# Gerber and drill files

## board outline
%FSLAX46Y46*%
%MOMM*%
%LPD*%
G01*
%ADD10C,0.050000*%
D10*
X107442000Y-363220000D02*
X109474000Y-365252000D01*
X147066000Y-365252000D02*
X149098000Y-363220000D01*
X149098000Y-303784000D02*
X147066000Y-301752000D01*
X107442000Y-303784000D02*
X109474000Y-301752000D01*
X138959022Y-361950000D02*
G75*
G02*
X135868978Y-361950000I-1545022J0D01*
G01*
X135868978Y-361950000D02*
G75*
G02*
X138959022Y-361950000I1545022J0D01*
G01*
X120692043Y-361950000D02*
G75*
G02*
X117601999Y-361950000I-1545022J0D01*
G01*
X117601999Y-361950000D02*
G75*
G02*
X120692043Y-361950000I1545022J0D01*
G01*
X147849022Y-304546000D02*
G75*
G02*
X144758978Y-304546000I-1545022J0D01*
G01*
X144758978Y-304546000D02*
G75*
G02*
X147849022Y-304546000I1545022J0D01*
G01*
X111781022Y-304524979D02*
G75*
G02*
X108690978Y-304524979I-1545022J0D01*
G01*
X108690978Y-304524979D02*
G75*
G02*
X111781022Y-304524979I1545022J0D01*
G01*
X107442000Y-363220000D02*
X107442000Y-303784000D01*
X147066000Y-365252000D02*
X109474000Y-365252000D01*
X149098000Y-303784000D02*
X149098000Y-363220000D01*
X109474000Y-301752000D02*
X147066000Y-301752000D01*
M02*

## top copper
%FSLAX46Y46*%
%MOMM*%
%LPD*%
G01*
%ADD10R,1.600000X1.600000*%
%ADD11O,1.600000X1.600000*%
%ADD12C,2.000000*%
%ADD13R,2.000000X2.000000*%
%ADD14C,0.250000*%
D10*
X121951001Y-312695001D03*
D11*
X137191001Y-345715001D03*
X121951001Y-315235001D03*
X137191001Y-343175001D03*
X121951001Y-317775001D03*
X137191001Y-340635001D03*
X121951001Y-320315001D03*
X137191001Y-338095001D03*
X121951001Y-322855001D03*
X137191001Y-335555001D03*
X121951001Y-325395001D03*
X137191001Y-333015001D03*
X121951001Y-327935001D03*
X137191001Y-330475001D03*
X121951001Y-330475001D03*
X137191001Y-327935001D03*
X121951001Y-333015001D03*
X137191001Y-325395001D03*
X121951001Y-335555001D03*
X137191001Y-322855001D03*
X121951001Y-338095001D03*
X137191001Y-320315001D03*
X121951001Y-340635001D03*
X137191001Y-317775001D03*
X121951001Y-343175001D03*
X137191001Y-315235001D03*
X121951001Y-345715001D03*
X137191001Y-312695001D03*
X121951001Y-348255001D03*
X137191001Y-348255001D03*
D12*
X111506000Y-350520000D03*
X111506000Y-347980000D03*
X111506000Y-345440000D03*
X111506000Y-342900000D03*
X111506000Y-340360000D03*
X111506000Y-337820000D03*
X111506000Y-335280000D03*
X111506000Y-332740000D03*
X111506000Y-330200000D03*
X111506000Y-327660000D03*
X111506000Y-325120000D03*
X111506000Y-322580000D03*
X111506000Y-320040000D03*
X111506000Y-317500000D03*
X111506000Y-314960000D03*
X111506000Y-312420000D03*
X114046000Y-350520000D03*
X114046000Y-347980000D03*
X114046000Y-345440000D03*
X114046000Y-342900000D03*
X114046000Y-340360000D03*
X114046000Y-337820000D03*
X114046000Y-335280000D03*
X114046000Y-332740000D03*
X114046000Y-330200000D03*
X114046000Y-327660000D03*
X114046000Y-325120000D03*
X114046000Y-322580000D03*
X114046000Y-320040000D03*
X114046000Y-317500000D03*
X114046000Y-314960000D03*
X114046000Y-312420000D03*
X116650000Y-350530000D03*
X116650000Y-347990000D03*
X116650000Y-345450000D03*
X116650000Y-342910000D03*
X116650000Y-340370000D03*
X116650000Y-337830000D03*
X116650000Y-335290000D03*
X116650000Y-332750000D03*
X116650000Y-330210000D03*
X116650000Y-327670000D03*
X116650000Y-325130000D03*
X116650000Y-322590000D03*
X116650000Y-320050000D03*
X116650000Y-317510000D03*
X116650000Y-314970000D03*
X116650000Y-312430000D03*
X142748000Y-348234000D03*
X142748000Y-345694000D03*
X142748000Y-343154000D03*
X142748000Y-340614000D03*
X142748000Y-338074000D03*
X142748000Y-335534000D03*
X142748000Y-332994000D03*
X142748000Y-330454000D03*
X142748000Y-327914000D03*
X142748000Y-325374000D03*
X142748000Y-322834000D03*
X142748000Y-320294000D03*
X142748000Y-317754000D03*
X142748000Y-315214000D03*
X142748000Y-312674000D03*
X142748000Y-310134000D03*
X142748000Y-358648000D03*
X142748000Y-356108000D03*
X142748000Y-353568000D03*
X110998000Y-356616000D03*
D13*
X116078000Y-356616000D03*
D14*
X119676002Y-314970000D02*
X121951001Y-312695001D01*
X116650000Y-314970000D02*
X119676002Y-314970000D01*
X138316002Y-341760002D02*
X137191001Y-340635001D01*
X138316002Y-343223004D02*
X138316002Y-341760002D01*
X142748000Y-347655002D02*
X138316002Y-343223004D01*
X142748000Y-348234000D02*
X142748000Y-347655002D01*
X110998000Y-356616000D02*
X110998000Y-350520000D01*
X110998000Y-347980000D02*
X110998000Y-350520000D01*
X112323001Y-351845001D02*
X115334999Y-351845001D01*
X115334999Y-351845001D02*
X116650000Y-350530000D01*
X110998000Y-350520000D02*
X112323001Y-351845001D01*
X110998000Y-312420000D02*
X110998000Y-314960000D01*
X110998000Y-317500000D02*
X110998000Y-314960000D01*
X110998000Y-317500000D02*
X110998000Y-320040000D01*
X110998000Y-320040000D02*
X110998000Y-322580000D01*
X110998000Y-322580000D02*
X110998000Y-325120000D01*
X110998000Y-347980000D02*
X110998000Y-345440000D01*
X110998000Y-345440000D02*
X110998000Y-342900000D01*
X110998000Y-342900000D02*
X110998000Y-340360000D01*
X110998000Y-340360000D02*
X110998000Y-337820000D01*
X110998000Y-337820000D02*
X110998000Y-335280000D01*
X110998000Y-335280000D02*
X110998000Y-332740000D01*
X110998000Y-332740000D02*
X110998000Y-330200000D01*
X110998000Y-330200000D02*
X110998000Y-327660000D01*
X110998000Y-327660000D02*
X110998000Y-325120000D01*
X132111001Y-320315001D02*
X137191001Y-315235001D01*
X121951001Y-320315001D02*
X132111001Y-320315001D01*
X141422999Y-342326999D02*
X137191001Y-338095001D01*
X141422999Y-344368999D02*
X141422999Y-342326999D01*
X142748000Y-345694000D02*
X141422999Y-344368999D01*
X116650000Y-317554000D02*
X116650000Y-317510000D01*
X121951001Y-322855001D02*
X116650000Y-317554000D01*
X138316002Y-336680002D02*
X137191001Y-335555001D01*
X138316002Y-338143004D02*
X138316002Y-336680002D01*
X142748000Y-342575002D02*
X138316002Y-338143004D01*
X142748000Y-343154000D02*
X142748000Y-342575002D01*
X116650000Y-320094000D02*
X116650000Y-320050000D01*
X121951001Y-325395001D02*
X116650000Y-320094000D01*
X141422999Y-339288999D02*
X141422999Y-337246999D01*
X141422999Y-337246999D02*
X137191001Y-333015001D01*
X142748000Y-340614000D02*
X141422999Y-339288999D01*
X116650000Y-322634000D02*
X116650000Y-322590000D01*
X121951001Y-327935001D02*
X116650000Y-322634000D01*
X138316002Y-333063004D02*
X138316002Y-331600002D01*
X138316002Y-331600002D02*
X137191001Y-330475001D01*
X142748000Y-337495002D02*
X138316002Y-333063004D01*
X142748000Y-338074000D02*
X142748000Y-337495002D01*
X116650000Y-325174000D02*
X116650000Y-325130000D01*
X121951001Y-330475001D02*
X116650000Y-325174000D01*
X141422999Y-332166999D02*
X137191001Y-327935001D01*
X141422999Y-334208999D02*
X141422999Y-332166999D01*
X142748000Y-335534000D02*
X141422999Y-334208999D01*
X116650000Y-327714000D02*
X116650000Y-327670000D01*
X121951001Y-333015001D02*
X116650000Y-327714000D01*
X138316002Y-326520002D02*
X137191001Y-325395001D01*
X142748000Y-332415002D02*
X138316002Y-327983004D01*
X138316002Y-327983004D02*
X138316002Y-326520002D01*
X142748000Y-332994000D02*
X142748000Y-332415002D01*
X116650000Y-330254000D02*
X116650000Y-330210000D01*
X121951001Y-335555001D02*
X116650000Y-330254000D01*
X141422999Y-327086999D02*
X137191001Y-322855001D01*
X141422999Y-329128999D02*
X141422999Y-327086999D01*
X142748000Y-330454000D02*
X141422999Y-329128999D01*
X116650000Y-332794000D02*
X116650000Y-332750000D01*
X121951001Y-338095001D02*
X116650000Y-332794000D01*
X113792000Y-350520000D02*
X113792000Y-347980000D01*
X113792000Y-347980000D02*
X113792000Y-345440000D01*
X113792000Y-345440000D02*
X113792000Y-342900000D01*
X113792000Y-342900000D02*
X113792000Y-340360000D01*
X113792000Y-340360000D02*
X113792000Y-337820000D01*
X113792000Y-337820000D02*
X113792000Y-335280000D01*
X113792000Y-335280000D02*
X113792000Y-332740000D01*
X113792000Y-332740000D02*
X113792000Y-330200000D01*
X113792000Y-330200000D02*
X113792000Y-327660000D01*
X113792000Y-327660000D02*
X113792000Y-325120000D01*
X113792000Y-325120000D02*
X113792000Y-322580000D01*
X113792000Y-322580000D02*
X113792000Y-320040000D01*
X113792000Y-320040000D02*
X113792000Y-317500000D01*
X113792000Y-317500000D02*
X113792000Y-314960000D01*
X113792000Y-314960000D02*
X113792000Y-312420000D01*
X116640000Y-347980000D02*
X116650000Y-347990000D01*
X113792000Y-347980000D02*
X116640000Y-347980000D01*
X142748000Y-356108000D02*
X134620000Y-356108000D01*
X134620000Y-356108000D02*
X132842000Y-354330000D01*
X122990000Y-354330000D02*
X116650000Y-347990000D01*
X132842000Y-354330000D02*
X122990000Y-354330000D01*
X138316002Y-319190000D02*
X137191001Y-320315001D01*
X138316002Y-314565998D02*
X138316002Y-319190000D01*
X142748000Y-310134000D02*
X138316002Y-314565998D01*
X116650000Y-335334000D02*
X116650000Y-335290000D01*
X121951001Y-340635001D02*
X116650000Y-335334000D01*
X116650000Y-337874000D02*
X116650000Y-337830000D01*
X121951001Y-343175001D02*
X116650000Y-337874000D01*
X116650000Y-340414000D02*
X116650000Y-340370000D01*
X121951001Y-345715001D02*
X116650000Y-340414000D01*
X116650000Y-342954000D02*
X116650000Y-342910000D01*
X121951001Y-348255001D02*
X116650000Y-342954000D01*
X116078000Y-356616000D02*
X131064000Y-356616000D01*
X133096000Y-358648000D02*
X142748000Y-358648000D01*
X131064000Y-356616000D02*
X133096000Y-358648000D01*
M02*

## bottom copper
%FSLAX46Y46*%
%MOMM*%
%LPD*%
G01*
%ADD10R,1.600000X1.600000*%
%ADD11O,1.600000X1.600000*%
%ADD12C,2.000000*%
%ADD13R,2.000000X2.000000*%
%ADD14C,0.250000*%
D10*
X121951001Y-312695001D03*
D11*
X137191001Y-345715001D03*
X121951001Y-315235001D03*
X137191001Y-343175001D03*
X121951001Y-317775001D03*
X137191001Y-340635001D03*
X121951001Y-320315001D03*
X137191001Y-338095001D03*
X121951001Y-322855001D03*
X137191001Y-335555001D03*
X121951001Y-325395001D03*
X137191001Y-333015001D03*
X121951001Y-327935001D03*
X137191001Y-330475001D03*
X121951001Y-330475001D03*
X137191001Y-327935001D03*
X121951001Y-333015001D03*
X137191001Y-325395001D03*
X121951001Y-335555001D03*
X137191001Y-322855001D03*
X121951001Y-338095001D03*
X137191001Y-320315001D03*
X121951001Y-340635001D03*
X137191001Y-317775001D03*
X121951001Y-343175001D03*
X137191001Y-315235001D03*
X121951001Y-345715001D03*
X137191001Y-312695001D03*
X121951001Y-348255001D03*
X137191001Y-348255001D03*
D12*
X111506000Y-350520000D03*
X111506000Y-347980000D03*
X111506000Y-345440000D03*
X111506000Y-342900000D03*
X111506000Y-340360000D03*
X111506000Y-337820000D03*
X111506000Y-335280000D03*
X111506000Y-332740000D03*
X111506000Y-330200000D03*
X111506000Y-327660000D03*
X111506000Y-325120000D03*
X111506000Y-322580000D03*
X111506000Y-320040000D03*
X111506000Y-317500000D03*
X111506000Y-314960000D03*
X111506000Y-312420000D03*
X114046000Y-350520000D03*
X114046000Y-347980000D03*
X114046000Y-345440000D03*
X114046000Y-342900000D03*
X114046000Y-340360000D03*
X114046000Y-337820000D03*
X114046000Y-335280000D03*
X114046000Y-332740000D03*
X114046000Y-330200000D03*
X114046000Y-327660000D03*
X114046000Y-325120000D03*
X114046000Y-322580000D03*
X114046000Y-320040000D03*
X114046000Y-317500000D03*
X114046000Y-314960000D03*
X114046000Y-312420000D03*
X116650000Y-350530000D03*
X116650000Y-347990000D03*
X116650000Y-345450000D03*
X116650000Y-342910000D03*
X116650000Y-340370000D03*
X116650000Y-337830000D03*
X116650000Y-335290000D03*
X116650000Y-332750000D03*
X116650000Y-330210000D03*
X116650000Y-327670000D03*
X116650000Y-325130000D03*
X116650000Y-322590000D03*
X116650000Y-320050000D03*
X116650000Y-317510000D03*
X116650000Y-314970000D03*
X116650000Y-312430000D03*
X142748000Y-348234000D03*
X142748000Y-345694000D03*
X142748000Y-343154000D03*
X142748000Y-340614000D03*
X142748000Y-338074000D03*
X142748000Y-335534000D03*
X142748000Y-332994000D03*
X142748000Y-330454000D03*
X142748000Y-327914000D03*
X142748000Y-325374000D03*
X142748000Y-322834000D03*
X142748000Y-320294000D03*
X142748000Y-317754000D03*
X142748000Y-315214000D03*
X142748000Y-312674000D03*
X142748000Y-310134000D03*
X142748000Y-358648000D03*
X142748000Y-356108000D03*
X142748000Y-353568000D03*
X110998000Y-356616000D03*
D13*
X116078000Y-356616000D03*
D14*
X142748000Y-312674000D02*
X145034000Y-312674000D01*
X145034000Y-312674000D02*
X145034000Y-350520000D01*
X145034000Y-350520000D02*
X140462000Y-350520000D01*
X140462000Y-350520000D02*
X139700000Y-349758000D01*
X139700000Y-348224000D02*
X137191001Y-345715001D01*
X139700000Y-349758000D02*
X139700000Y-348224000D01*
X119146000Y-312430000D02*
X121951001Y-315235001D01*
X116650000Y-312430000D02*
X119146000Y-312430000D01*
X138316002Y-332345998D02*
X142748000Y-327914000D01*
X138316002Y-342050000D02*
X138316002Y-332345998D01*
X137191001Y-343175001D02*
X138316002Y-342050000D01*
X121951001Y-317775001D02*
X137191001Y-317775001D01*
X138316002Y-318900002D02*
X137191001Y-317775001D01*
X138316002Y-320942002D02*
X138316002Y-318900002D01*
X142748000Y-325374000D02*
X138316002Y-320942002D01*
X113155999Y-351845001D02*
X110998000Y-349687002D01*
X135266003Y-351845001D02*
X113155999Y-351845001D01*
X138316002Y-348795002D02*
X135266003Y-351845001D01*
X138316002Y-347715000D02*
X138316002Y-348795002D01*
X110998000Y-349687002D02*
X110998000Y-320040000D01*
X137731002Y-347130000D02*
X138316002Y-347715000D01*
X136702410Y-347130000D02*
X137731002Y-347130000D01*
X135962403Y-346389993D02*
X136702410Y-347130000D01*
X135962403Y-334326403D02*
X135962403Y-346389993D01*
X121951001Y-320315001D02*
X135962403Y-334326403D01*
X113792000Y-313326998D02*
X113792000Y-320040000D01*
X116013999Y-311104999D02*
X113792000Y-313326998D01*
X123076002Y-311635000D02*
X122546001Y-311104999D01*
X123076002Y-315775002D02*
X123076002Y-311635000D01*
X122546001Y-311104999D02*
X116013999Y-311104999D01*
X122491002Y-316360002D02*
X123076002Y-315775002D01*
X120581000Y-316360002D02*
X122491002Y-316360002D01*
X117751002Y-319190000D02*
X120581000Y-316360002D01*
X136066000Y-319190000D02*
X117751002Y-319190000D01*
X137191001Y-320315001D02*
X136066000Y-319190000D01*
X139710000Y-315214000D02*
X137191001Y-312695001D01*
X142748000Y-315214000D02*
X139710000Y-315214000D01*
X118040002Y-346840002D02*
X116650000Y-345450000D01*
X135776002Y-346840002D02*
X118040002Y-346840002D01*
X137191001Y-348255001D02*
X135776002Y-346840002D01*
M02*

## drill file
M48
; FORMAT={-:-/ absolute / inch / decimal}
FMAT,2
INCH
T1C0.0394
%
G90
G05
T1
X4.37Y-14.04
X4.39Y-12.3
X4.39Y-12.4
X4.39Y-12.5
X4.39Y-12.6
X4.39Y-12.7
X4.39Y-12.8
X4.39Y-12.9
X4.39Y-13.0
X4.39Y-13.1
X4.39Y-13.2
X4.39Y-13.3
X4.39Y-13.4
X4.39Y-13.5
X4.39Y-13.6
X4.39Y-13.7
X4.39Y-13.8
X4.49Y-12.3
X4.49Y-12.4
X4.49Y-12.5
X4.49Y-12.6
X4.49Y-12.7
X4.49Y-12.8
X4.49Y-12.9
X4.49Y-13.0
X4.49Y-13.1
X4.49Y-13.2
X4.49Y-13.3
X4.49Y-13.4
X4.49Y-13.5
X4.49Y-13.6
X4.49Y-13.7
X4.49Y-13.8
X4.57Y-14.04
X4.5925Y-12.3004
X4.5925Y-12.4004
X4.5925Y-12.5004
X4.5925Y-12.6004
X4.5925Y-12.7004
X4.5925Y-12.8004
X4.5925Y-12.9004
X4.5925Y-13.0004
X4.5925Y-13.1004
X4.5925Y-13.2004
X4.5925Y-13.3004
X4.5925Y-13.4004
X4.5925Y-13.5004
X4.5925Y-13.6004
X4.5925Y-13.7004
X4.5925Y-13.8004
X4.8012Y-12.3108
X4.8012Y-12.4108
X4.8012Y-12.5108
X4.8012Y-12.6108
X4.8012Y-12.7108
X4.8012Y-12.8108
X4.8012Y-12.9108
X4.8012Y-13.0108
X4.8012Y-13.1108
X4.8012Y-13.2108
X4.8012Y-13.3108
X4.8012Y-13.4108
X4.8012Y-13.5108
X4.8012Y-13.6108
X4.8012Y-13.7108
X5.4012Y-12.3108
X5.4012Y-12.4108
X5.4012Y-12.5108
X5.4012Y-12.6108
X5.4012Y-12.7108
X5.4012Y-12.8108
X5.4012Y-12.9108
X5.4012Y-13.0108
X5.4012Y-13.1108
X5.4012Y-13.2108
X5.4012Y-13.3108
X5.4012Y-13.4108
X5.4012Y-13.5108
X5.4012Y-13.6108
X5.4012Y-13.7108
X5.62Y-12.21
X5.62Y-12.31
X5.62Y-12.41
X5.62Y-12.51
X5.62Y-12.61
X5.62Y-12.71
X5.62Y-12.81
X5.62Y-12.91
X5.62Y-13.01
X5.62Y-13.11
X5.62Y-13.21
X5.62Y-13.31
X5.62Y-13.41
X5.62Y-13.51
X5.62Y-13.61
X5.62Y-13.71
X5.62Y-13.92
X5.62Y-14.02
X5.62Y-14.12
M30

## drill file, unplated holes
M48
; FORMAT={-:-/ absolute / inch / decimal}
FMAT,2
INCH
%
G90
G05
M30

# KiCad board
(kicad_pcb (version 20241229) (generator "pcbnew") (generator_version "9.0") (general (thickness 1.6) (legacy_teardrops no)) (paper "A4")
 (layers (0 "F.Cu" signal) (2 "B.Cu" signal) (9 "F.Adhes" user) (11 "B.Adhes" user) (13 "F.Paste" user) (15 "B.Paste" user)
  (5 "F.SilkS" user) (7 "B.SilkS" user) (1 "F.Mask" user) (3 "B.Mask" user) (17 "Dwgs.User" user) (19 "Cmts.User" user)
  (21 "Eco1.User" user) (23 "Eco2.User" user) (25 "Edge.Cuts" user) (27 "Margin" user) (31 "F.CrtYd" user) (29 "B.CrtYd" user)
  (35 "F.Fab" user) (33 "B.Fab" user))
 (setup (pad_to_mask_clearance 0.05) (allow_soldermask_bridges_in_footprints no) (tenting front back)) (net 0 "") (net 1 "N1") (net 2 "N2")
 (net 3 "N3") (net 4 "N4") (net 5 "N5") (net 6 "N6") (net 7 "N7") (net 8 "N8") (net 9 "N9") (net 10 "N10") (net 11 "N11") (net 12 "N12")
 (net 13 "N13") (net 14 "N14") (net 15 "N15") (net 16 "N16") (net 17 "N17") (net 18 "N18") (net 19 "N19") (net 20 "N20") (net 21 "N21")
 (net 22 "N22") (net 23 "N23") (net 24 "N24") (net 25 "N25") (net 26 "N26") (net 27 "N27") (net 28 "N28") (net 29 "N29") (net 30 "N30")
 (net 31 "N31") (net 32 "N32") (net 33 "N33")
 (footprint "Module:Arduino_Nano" (layer "F.Cu") (at 121.951001 312.695001)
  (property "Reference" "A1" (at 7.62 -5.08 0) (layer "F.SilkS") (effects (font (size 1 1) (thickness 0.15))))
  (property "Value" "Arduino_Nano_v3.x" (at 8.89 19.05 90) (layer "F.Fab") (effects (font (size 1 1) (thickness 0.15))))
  (pad "1" thru_hole rect (at 0 0) (size 1.6 1.6) (drill 1) (layers "*.Cu" "*.Mask") (remove_unused_layers no) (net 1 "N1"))
  (pad "2" thru_hole oval (at 0 2.54) (size 1.6 1.6) (drill 1) (layers "*.Cu" "*.Mask") (remove_unused_layers no) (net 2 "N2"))
  (pad "3" thru_hole oval (at 0 5.08) (size 1.6 1.6) (drill 1) (layers "*.Cu" "*.Mask") (remove_unused_layers no) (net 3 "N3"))
  (pad "4" thru_hole oval (at 0 7.62) (size 1.6 1.6) (drill 1) (layers "*.Cu" "*.Mask") (remove_unused_layers no) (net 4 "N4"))
  (pad "5" thru_hole oval (at 0 10.16) (size 1.6 1.6) (drill 1) (layers "*.Cu" "*.Mask") (remove_unused_layers no) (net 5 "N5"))
  (pad "6" thru_hole oval (at 0 12.7) (size 1.6 1.6) (drill 1) (layers "*.Cu" "*.Mask") (remove_unused_layers no) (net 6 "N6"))
  (pad "7" thru_hole oval (at 0 15.24) (size 1.6 1.6) (drill 1) (layers "*.Cu" "*.Mask") (remove_unused_layers no) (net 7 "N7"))
  (pad "8" thru_hole oval (at 0 17.78) (size 1.6 1.6) (drill 1) (layers "*.Cu" "*.Mask") (remove_unused_layers no) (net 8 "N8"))
  (pad "9" thru_hole oval (at 0 20.32) (size 1.6 1.6) (drill 1) (layers "*.Cu" "*.Mask") (remove_unused_layers no) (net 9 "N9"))
  (pad "10" thru_hole oval (at 0 22.86) (size 1.6 1.6) (drill 1) (layers "*.Cu" "*.Mask") (remove_unused_layers no) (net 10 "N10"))
  (pad "11" thru_hole oval (at 0 25.4) (size 1.6 1.6) (drill 1) (layers "*.Cu" "*.Mask") (remove_unused_layers no) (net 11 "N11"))
  (pad "12" thru_hole oval (at 0 27.94) (size 1.6 1.6) (drill 1) (layers "*.Cu" "*.Mask") (remove_unused_layers no) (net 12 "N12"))
  (pad "13" thru_hole oval (at 0 30.48) (size 1.6 1.6) (drill 1) (layers "*.Cu" "*.Mask") (remove_unused_layers no) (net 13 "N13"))
  (pad "14" thru_hole oval (at 0 33.02) (size 1.6 1.6) (drill 1) (layers "*.Cu" "*.Mask") (remove_unused_layers no) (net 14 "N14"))
  (pad "15" thru_hole oval (at 0 35.56) (size 1.6 1.6) (drill 1) (layers "*.Cu" "*.Mask") (remove_unused_layers no) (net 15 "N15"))
  (pad "16" thru_hole oval (at 15.24 35.56) (size 1.6 1.6) (drill 1) (layers "*.Cu" "*.Mask") (remove_unused_layers no) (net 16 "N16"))
  (pad "17" thru_hole oval (at 15.24 33.02) (size 1.6 1.6) (drill 1) (layers "*.Cu" "*.Mask") (remove_unused_layers no) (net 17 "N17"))
  (pad "18" thru_hole oval (at 15.24 30.48) (size 1.6 1.6) (drill 1) (layers "*.Cu" "*.Mask") (remove_unused_layers no) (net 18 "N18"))
  (pad "19" thru_hole oval (at 15.24 27.94) (size 1.6 1.6) (drill 1) (layers "*.Cu" "*.Mask") (remove_unused_layers no) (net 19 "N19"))
  (pad "20" thru_hole oval (at 15.24 25.4) (size 1.6 1.6) (drill 1) (layers "*.Cu" "*.Mask") (remove_unused_layers no) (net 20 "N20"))
  (pad "21" thru_hole oval (at 15.24 22.86) (size 1.6 1.6) (drill 1) (layers "*.Cu" "*.Mask") (remove_unused_layers no) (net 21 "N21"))
  (pad "22" thru_hole oval (at 15.24 20.32) (size 1.6 1.6) (drill 1) (layers "*.Cu" "*.Mask") (remove_unused_layers no) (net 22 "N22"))
  (pad "23" thru_hole oval (at 15.24 17.78) (size 1.6 1.6) (drill 1) (layers "*.Cu" "*.Mask") (remove_unused_layers no) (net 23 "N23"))
  (pad "24" thru_hole oval (at 15.24 15.24) (size 1.6 1.6) (drill 1) (layers "*.Cu" "*.Mask") (remove_unused_layers no) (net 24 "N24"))
  (pad "25" thru_hole oval (at 15.24 12.7) (size 1.6 1.6) (drill 1) (layers "*.Cu" "*.Mask") (remove_unused_layers no) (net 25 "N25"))
  (pad "26" thru_hole oval (at 15.24 10.16) (size 1.6 1.6) (drill 1) (layers "*.Cu" "*.Mask") (remove_unused_layers no) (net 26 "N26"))
  (pad "27" thru_hole oval (at 15.24 7.62) (size 1.6 1.6) (drill 1) (layers "*.Cu" "*.Mask") (remove_unused_layers no) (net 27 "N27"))
  (pad "28" thru_hole oval (at 15.24 5.08) (size 1.6 1.6) (drill 1) (layers "*.Cu" "*.Mask") (remove_unused_layers no) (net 3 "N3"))
  (pad "29" thru_hole oval (at 15.24 2.54) (size 1.6 1.6) (drill 1) (layers "*.Cu" "*.Mask") (remove_unused_layers no) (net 4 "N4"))
  (pad "30" thru_hole oval (at 15.24 0) (size 1.6 1.6) (drill 1) (layers "*.Cu" "*.Mask") (remove_unused_layers no) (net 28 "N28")))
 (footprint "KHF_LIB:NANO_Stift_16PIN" (layer "F.Cu") (at 114.046 312.42 -90)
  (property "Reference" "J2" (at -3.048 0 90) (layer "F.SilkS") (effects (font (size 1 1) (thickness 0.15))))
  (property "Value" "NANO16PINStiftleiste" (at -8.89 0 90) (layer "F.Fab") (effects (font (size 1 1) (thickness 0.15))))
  (pad "1" thru_hole circle (at 0 0 270) (size 2 2) (drill 1) (layers "*.Cu" "*.Mask") (remove_unused_layers no) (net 27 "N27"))
  (pad "2" thru_hole circle (at 2.54 0 270) (size 2 2) (drill 1) (layers "*.Cu" "*.Mask") (remove_unused_layers no) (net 27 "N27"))
  (pad "3" thru_hole circle (at 5.08 0 270) (size 2 2) (drill 1) (layers "*.Cu" "*.Mask") (remove_unused_layers no) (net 27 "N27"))
  (pad "4" thru_hole circle (at 7.62 0 270) (size 2 2) (drill 1) (layers "*.Cu" "*.Mask") (remove_unused_layers no) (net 27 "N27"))
  (pad "5" thru_hole circle (at 10.16 0 270) (size 2 2) (drill 1) (layers "*.Cu" "*.Mask") (remove_unused_layers no) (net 27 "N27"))
  (pad "6" thru_hole circle (at 12.7 0 270) (size 2 2) (drill 1) (layers "*.Cu" "*.Mask") (remove_unused_layers no) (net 27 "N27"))
  (pad "7" thru_hole circle (at 15.24 0 270) (size 2 2) (drill 1) (layers "*.Cu" "*.Mask") (remove_unused_layers no) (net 27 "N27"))
  (pad "8" thru_hole circle (at 17.78 0 270) (size 2 2) (drill 1) (layers "*.Cu" "*.Mask") (remove_unused_layers no) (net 27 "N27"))
  (pad "9" thru_hole circle (at 20.32 0 270) (size 2 2) (drill 1) (layers "*.Cu" "*.Mask") (remove_unused_layers no) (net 27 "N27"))
  (pad "10" thru_hole circle (at 22.86 0 270) (size 2 2) (drill 1) (layers "*.Cu" "*.Mask") (remove_unused_layers no) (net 27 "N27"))
  (pad "11" thru_hole circle (at 25.4 0 270) (size 2 2) (drill 1) (layers "*.Cu" "*.Mask") (remove_unused_layers no) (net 27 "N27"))
  (pad "12" thru_hole circle (at 27.94 0 270) (size 2 2) (drill 1) (layers "*.Cu" "*.Mask") (remove_unused_layers no) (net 27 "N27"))
  (pad "13" thru_hole circle (at 30.48 0 270) (size 2 2) (drill 1) (layers "*.Cu" "*.Mask") (remove_unused_layers no) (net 27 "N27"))
  (pad "14" thru_hole circle (at 33.02 0 270) (size 2 2) (drill 1) (layers "*.Cu" "*.Mask") (remove_unused_layers no) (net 27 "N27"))
  (pad "15" thru_hole circle (at 35.56 0 270) (size 2 2) (drill 1) (layers "*.Cu" "*.Mask") (remove_unused_layers no) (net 27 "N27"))
  (pad "16" thru_hole circle (at 38.1 0 270) (size 2 2) (drill 1) (layers "*.Cu" "*.Mask") (remove_unused_layers no) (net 27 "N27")))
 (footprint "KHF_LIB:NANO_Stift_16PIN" (layer "F.Cu") (at 116.65 312.43 -90)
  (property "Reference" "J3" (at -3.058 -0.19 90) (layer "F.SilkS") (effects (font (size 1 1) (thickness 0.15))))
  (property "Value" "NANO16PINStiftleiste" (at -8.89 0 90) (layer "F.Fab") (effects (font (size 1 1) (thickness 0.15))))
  (pad "1" thru_hole circle (at 0 0 270) (size 2 2) (drill 1) (layers "*.Cu" "*.Mask") (remove_unused_layers no) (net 2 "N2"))
  (pad "2" thru_hole circle (at 2.54 0 270) (size 2 2) (drill 1) (layers "*.Cu" "*.Mask") (remove_unused_layers no) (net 1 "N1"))
  (pad "3" thru_hole circle (at 5.08 0 270) (size 2 2) (drill 1) (layers "*.Cu" "*.Mask") (remove_unused_layers no) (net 5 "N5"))
  (pad "4" thru_hole circle (at 7.62 0 270) (size 2 2) (drill 1) (layers "*.Cu" "*.Mask") (remove_unused_layers no) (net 6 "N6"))
  (pad "5" thru_hole circle (at 10.16 0 270) (size 2 2) (drill 1) (layers "*.Cu" "*.Mask") (remove_unused_layers no) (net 7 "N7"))
  (pad "6" thru_hole circle (at 12.7 0 270) (size 2 2) (drill 1) (layers "*.Cu" "*.Mask") (remove_unused_layers no) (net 8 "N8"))
  (pad "7" thru_hole circle (at 15.24 0 270) (size 2 2) (drill 1) (layers "*.Cu" "*.Mask") (remove_unused_layers no) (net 9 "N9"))
  (pad "8" thru_hole circle (at 17.78 0 270) (size 2 2) (drill 1) (layers "*.Cu" "*.Mask") (remove_unused_layers no) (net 10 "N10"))
  (pad "9" thru_hole circle (at 20.32 0 270) (size 2 2) (drill 1) (layers "*.Cu" "*.Mask") (remove_unused_layers no) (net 11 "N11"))
  (pad "10" thru_hole circle (at 22.86 0 270) (size 2 2) (drill 1) (layers "*.Cu" "*.Mask") (remove_unused_layers no) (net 12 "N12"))
  (pad "11" thru_hole circle (at 25.4 0 270) (size 2 2) (drill 1) (layers "*.Cu" "*.Mask") (remove_unused_layers no) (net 13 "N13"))
  (pad "12" thru_hole circle (at 27.94 0 270) (size 2 2) (drill 1) (layers "*.Cu" "*.Mask") (remove_unused_layers no) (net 14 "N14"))
  (pad "13" thru_hole circle (at 30.48 0 270) (size 2 2) (drill 1) (layers "*.Cu" "*.Mask") (remove_unused_layers no) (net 15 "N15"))
  (pad "14" thru_hole circle (at 33.02 0 270) (size 2 2) (drill 1) (layers "*.Cu" "*.Mask") (remove_unused_layers no) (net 16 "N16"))
  (pad "15" thru_hole circle (at 35.56 0 270) (size 2 2) (drill 1) (layers "*.Cu" "*.Mask") (remove_unused_layers no) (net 27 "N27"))
  (pad "16" thru_hole circle (at 38.1 0 270) (size 2 2) (drill 1) (layers "*.Cu" "*.Mask") (remove_unused_layers no) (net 4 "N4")))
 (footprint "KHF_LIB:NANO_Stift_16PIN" (layer "F.Cu") (at 142.748 348.234 90)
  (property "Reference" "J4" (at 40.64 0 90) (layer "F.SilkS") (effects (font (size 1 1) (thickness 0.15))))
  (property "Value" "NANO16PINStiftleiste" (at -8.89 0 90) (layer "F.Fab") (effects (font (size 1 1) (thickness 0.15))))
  (pad "1" thru_hole circle (at 0 0 90) (size 2 2) (drill 1) (layers "*.Cu" "*.Mask") (remove_unused_layers no) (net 19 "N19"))
  (pad "2" thru_hole circle (at 2.54 0 90) (size 2 2) (drill 1) (layers "*.Cu" "*.Mask") (remove_unused_layers no) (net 20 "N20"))
  (pad "3" thru_hole circle (at 5.08 0 90) (size 2 2) (drill 1) (layers "*.Cu" "*.Mask") (remove_unused_layers no) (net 21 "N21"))
  (pad "4" thru_hole circle (at 7.62 0 90) (size 2 2) (drill 1) (layers "*.Cu" "*.Mask") (remove_unused_layers no) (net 22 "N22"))
  (pad "5" thru_hole circle (at 10.16 0 90) (size 2 2) (drill 1) (layers "*.Cu" "*.Mask") (remove_unused_layers no) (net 23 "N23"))
  (pad "6" thru_hole circle (at 12.7 0 90) (size 2 2) (drill 1) (layers "*.Cu" "*.Mask") (remove_unused_layers no) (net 24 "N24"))
  (pad "7" thru_hole circle (at 15.24 0 90) (size 2 2) (drill 1) (layers "*.Cu" "*.Mask") (remove_unused_layers no) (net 25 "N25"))
  (pad "8" thru_hole circle (at 17.78 0 90) (size 2 2) (drill 1) (layers "*.Cu" "*.Mask") (remove_unused_layers no) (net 26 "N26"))
  (pad "9" thru_hole circle (at 20.32 0 90) (size 2 2) (drill 1) (layers "*.Cu" "*.Mask") (remove_unused_layers no) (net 18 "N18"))
  (pad "10" thru_hole circle (at 22.86 0 90) (size 2 2) (drill 1) (layers "*.Cu" "*.Mask") (remove_unused_layers no) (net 3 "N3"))
  (pad "11" thru_hole circle (at 25.4 0 90) (size 2 2) (drill 1) (layers "*.Cu" "*.Mask") (remove_unused_layers no) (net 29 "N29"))
  (pad "12" thru_hole circle (at 27.94 0 90) (size 2 2) (drill 1) (layers "*.Cu" "*.Mask") (remove_unused_layers no) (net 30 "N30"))
  (pad "13" thru_hole circle (at 30.48 0 90) (size 2 2) (drill 1) (layers "*.Cu" "*.Mask") (remove_unused_layers no) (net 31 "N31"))
  (pad "14" thru_hole circle (at 33.02 0 90) (size 2 2) (drill 1) (layers "*.Cu" "*.Mask") (remove_unused_layers no) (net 28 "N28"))
  (pad "15" thru_hole circle (at 35.56 0 90) (size 2 2) (drill 1) (layers "*.Cu" "*.Mask") (remove_unused_layers no) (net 17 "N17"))
  (pad "16" thru_hole circle (at 38.1 0 90) (size 2 2) (drill 1) (layers "*.Cu" "*.Mask") (remove_unused_layers no) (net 27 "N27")))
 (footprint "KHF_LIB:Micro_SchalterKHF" (layer "F.Cu") (at 142.748 358.648 90)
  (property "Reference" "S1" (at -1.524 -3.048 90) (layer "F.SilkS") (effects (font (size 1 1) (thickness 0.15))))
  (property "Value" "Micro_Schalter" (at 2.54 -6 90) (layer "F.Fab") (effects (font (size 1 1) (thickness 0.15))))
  (pad "1" thru_hole circle (at 0 0 90) (size 2 2) (drill 1) (layers "*.Cu" "*.Mask") (remove_unused_layers no) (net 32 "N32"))
  (pad "2" thru_hole circle (at 2.54 0 90) (size 2 2) (drill 1) (layers "*.Cu" "*.Mask") (remove_unused_layers no) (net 27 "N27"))
  (pad "3" thru_hole circle (at 5.08 0 90) (size 2 2) (drill 1) (layers "*.Cu" "*.Mask") (remove_unused_layers no) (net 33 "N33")))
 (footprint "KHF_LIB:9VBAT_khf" (layer "F.Cu") (at 110.998 356.616)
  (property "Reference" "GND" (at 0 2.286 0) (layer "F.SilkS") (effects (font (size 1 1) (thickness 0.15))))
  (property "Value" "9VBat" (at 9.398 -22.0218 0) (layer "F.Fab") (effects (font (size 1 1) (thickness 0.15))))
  (pad "1" thru_hole circle (at 0 0) (size 2 2) (drill 1) (layers "*.Cu" "*.Mask") (remove_unused_layers no) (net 4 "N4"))
  (pad "2" thru_hole rect (at 5.08 0) (size 2 2) (drill 1) (layers "*.Cu" "*.Mask") (remove_unused_layers no) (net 32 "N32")))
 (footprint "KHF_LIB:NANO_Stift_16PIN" (layer "F.Cu") (at 111.506 350.52 90)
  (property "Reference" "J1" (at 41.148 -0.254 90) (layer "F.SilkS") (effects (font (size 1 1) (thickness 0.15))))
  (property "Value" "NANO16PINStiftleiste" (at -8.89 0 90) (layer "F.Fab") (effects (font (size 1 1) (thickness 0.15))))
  (pad "1" thru_hole circle (at 0 0 90) (size 2 2) (drill 1) (layers "*.Cu" "*.Mask") (remove_unused_layers no) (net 4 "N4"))
  (pad "2" thru_hole circle (at 2.54 0 90) (size 2 2) (drill 1) (layers "*.Cu" "*.Mask") (remove_unused_layers no) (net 4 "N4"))
  (pad "3" thru_hole circle (at 5.08 0 90) (size 2 2) (drill 1) (layers "*.Cu" "*.Mask") (remove_unused_layers no) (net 4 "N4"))
  (pad "4" thru_hole circle (at 7.62 0 90) (size 2 2) (drill 1) (layers "*.Cu" "*.Mask") (remove_unused_layers no) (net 4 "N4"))
  (pad "5" thru_hole circle (at 10.16 0 90) (size 2 2) (drill 1) (layers "*.Cu" "*.Mask") (remove_unused_layers no) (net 4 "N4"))
  (pad "6" thru_hole circle (at 12.7 0 90) (size 2 2) (drill 1) (layers "*.Cu" "*.Mask") (remove_unused_layers no) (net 4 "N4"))
  (pad "7" thru_hole circle (at 15.24 0 90) (size 2 2) (drill 1) (layers "*.Cu" "*.Mask") (remove_unused_layers no) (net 4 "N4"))
  (pad "8" thru_hole circle (at 17.78 0 90) (size 2 2) (drill 1) (layers "*.Cu" "*.Mask") (remove_unused_layers no) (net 4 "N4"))
  (pad "9" thru_hole circle (at 20.32 0 90) (size 2 2) (drill 1) (layers "*.Cu" "*.Mask") (remove_unused_layers no) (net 4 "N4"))
  (pad "10" thru_hole circle (at 22.86 0 90) (size 2 2) (drill 1) (layers "*.Cu" "*.Mask") (remove_unused_layers no) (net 4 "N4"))
  (pad "11" thru_hole circle (at 25.4 0 90) (size 2 2) (drill 1) (layers "*.Cu" "*.Mask") (remove_unused_layers no) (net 4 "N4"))
  (pad "12" thru_hole circle (at 27.94 0 90) (size 2 2) (drill 1) (layers "*.Cu" "*.Mask") (remove_unused_layers no) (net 4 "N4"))
  (pad "13" thru_hole circle (at 30.48 0 90) (size 2 2) (drill 1) (layers "*.Cu" "*.Mask") (remove_unused_layers no) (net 4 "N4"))
  (pad "14" thru_hole circle (at 33.02 0 90) (size 2 2) (drill 1) (layers "*.Cu" "*.Mask") (remove_unused_layers no) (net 4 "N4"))
  (pad "15" thru_hole circle (at 35.56 0 90) (size 2 2) (drill 1) (layers "*.Cu" "*.Mask") (remove_unused_layers no) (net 4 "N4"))
  (pad "16" thru_hole circle (at 38.1 0 90) (size 2 2) (drill 1) (layers "*.Cu" "*.Mask") (remove_unused_layers no) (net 4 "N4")))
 (gr_line (start 107.442 363.22) (end 107.442 303.784) (stroke (width 0.05) (type solid)) (layer "Edge.Cuts"))
 (gr_circle (center 137.414 361.95) (end 138.938 361.696) (stroke (width 0.05) (type solid)) (fill no) (layer "Edge.Cuts"))
 (gr_circle (center 146.304 304.546) (end 147.828 304.292) (stroke (width 0.05) (type solid)) (fill no) (layer "Edge.Cuts"))
 (gr_line (start 107.442 303.784) (end 109.474 301.752) (stroke (width 0.05) (type solid)) (layer "Edge.Cuts"))
 (gr_line (start 147.066 365.252) (end 149.098 363.22) (stroke (width 0.05) (type solid)) (layer "Edge.Cuts"))
 (gr_line (start 147.066 365.252) (end 109.474 365.252) (stroke (width 0.05) (type solid)) (layer "Edge.Cuts"))
 (gr_line (start 149.098 303.784) (end 149.098 363.22) (stroke (width 0.05) (type solid)) (layer "Edge.Cuts"))
 (gr_line (start 149.098 303.784) (end 147.066 301.752) (stroke (width 0.05) (type solid)) (layer "Edge.Cuts"))
 (gr_circle (center 119.147021 361.95) (end 120.671021 361.696) (stroke (width 0.05) (type solid)) (fill no) (layer "Edge.Cuts"))
 (gr_line (start 107.442 363.22) (end 109.474 365.252) (stroke (width 0.05) (type solid)) (layer "Edge.Cuts"))
 (gr_line (start 109.474 301.752) (end 147.066 301.752) (stroke (width 0.05) (type solid)) (layer "Edge.Cuts"))
 (gr_circle (center 110.236 304.524979) (end 111.76 304.270979) (stroke (width 0.05) (type solid)) (fill no) (layer "Edge.Cuts"))
 (segment (start 119.676002 314.97) (end 121.951001 312.695001) (width 0.25) (layer "F.Cu") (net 1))
 (segment (start 116.65 314.97) (end 119.676002 314.97) (width 0.25) (layer "F.Cu") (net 1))
 (segment (start 142.748 312.674) (end 145.034 312.674) (width 0.25) (layer "B.Cu") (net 17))
 (segment (start 145.034 350.52) (end 140.462 350.52) (width 0.25) (layer "B.Cu") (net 17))
 (segment (start 139.7 349.758) (end 139.7 348.224) (width 0.25) (layer "B.Cu") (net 17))
 (segment (start 140.462 350.52) (end 139.7 349.758) (width 0.25) (layer "B.Cu") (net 17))
 (segment (start 145.034 312.674) (end 145.034 350.52) (width 0.25) (layer "B.Cu") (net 17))
 (segment (start 139.7 348.224) (end 137.191001 345.715001) (width 0.25) (layer "B.Cu") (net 17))
 (segment (start 119.146 312.43) (end 121.951001 315.235001) (width 0.25) (layer "B.Cu") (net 2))
 (segment (start 116.65 312.43) (end 119.146 312.43) (width 0.25) (layer "B.Cu") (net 2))
 (segment (start 138.316002 332.345998) (end 142.748 327.914) (width 0.25) (layer "B.Cu") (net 18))
 (segment (start 138.316002 342.05) (end 138.316002 332.345998) (width 0.25) (layer "B.Cu") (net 18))
 (segment (start 137.191001 343.175001) (end 138.316002 342.05) (width 0.25) (layer "B.Cu") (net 18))
 (segment (start 138.316002 320.942002) (end 138.316002 318.900002) (width 0.25) (layer "B.Cu") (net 3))
 (segment (start 138.316002 318.900002) (end 137.191001 317.775001) (width 0.25) (layer "B.Cu") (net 3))
 (segment (start 142.748 325.374) (end 138.316002 320.942002) (width 0.25) (layer "B.Cu") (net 3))
 (segment (start 121.951001 317.775001) (end 137.191001 317.775001) (width 0.25) (layer "B.Cu") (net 3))
 (segment (start 142.748 347.655002) (end 138.316002 343.223004) (width 0.25) (layer "F.Cu") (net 19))
 (segment (start 138.316002 341.760002) (end 137.191001 340.635001) (width 0.25) (layer "F.Cu") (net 19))
 (segment (start 138.316002 343.223004) (end 138.316002 341.760002) (width 0.25) (layer "F.Cu") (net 19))
 (segment (start 142.748 348.234) (end 142.748 347.655002) (width 0.25) (layer "F.Cu") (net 19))
 (segment (start 110.998 356.616) (end 110.998 350.52) (width 0.25) (layer "F.Cu") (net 4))
 (segment (start 110.998 337.82) (end 110.998 335.28) (width 0.25) (layer "F.Cu") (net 4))
 (segment (start 110.998 322.58) (end 110.998 325.12) (width 0.25) (layer "F.Cu") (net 4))
 (segment (start 110.998 317.5) (end 110.998 314.96) (width 0.25) (layer "F.Cu") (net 4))
 (segment (start 110.998 347.98) (end 110.998 350.52) (width 0.25) (layer "F.Cu") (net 4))
 (segment (start 110.998 347.98) (end 110.998 345.44) (width 0.25) (layer "F.Cu") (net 4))
 (segment (start 115.334999 351.845001) (end 116.65 350.53) (width 0.25) (layer "F.Cu") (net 4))
 (segment (start 110.998 312.42) (end 110.998 314.96) (width 0.25) (layer "F.Cu") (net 4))
 (segment (start 132.111001 320.315001) (end 137.191001 315.235001) (width 0.25) (layer "F.Cu") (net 4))
 (segment (start 110.998 320.04) (end 110.998 322.58) (width 0.25) (layer "F.Cu") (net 4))
 (segment (start 110.998 342.9) (end 110.998 340.36) (width 0.25) (layer "F.Cu") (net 4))
 (segment (start 110.998 317.5) (end 110.998 320.04) (width 0.25) (layer "F.Cu") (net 4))
 (segment (start 110.998 332.74) (end 110.998 330.2) (width 0.25) (layer "F.Cu") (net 4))
 (segment (start 110.998 327.66) (end 110.998 325.12) (width 0.25) (layer "F.Cu") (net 4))
 (segment (start 110.998 330.2) (end 110.998 327.66) (width 0.25) (layer "F.Cu") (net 4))
 (segment (start 112.323001 351.845001) (end 115.334999 351.845001) (width 0.25) (layer "F.Cu") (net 4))
 (segment (start 110.998 345.44) (end 110.998 342.9) (width 0.25) (layer "F.Cu") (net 4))
 (segment (start 110.998 340.36) (end 110.998 337.82) (width 0.25) (layer "F.Cu") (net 4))
 (segment (start 121.951001 320.315001) (end 132.111001 320.315001) (width 0.25) (layer "F.Cu") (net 4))
 (segment (start 110.998 335.28) (end 110.998 332.74) (width 0.25) (layer "F.Cu") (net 4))
 (segment (start 110.998 350.52) (end 112.323001 351.845001) (width 0.25) (layer "F.Cu") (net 4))
 (segment (start 110.998 349.687002) (end 110.998 320.04) (width 0.25) (layer "B.Cu") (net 4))
 (segment (start 135.962403 334.326403) (end 135.962403 346.389993) (width 0.25) (layer "B.Cu") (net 4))
 (segment (start 135.266003 351.845001) (end 113.155999 351.845001) (width 0.25) (layer "B.Cu") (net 4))
 (segment (start 137.731002 347.13) (end 138.316002 347.715) (width 0.25) (layer "B.Cu") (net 4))
 (segment (start 135.962403 346.389993) (end 136.70241 347.13) (width 0.25) (layer "B.Cu") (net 4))
 (segment (start 136.70241 347.13) (end 137.731002 347.13) (width 0.25) (layer "B.Cu") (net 4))
 (segment (start 138.316002 347.715) (end 138.316002 348.795002) (width 0.25) (layer "B.Cu") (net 4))
 (segment (start 113.155999 351.845001) (end 110.998 349.687002) (width 0.25) (layer "B.Cu") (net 4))
 (segment (start 121.951001 320.315001) (end 135.962403 334.326403) (width 0.25) (layer "B.Cu") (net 4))
 (segment (start 138.316002 348.795002) (end 135.266003 351.845001) (width 0.25) (layer "B.Cu") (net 4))
 (segment (start 141.422999 342.326999) (end 137.191001 338.095001) (width 0.25) (layer "F.Cu") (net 20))
 (segment (start 142.748 345.694) (end 141.422999 344.368999) (width 0.25) (layer "F.Cu") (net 20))
 (segment (start 141.422999 344.368999) (end 141.422999 342.326999) (width 0.25) (layer "F.Cu") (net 20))
 (segment (start 116.65 317.554) (end 116.65 317.51) (width 0.25) (layer "F.Cu") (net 5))
 (segment (start 121.951001 322.855001) (end 116.65 317.554) (width 0.25) (layer "F.Cu") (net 5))
 (segment (start 142.748 343.154) (end 142.748 342.575002) (width 0.25) (layer "F.Cu") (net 21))
 (segment (start 142.748 342.575002) (end 138.316002 338.143004) (width 0.25) (layer "F.Cu") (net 21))
 (segment (start 138.316002 336.680002) (end 137.191001 335.555001) (width 0.25) (layer "F.Cu") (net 21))
 (segment (start 138.316002 338.143004) (end 138.316002 336.680002) (width 0.25) (layer "F.Cu") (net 21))
 (segment (start 121.951001 325.395001) (end 116.65 320.094) (width 0.25) (layer "F.Cu") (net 6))
 (segment (start 116.65 320.094) (end 116.65 320.05) (width 0.25) (layer "F.Cu") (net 6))
 (segment (start 141.422999 337.246999) (end 137.191001 333.015001) (width 0.25) (layer "F.Cu") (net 22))
 (segment (start 142.748 340.614) (end 141.422999 339.288999) (width 0.25) (layer "F.Cu") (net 22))
 (segment (start 141.422999 339.288999) (end 141.422999 337.246999) (width 0.25) (layer "F.Cu") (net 22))
 (segment (start 121.951001 327.935001) (end 116.65 322.634) (width 0.25) (layer "F.Cu") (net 7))
 (segment (start 116.65 322.634) (end 116.65 322.59) (width 0.25) (layer "F.Cu") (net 7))
 (segment (start 142.748 337.495002) (end 138.316002 333.063004) (width 0.25) (layer "F.Cu") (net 23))
 (segment (start 138.316002 331.600002) (end 137.191001 330.475001) (width 0.25) (layer "F.Cu") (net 23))
 (segment (start 138.316002 333.063004) (end 138.316002 331.600002) (width 0.25) (layer "F.Cu") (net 23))
 (segment (start 142.748 338.074) (end 142.748 337.495002) (width 0.25) (layer "F.Cu") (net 23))
 (segment (start 116.65 325.174) (end 116.65 325.13) (width 0.25) (layer "F.Cu") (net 8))
 (segment (start 121.951001 330.475001) (end 116.65 325.174) (width 0.25) (layer "F.Cu") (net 8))
 (segment (start 141.422999 332.166999) (end 137.191001 327.935001) (width 0.25) (layer "F.Cu") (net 24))
 (segment (start 142.748 335.534) (end 141.422999 334.208999) (width 0.25) (layer "F.Cu") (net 24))
 (segment (start 141.422999 334.208999) (end 141.422999 332.166999) (width 0.25) (layer "F.Cu") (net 24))
 (segment (start 116.65 327.714) (end 116.65 327.67) (width 0.25) (layer "F.Cu") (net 9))
 (segment (start 121.951001 333.015001) (end 116.65 327.714) (width 0.25) (layer "F.Cu") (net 9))
 (segment (start 142.748 332.994) (end 142.748 332.415002) (width 0.25) (layer "F.Cu") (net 25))
 (segment (start 138.316002 327.983004) (end 138.316002 326.520002) (width 0.25) (layer "F.Cu") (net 25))
 (segment (start 138.316002 326.520002) (end 137.191001 325.395001) (width 0.25) (layer "F.Cu") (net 25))
 (segment (start 142.748 332.415002) (end 138.316002 327.983004) (width 0.25) (layer "F.Cu") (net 25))
 (segment (start 116.65 330.254) (end 116.65 330.21) (width 0.25) (layer "F.Cu") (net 10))
 (segment (start 121.951001 335.555001) (end 116.65 330.254) (width 0.25) (layer "F.Cu") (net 10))
 (segment (start 141.422999 327.086999) (end 137.191001 322.855001) (width 0.25) (layer "F.Cu") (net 26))
 (segment (start 141.422999 329.128999) (end 141.422999 327.086999) (width 0.25) (layer "F.Cu") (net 26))
 (segment (start 142.748 330.454) (end 141.422999 329.128999) (width 0.25) (layer "F.Cu") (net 26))
 (segment (start 116.65 332.794) (end 116.65 332.75) (width 0.25) (layer "F.Cu") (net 11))
 (segment (start 121.951001 338.095001) (end 116.65 332.794) (width 0.25) (layer "F.Cu") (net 11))
 (segment (start 113.792 350.52) (end 113.792 347.98) (width 0.25) (layer "F.Cu") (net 27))
 (segment (start 113.792 327.66) (end 113.792 325.12) (width 0.25) (layer "F.Cu") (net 27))
 (segment (start 132.842 354.33) (end 122.99 354.33) (width 0.25) (layer "F.Cu") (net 27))
 (segment (start 113.792 314.96) (end 113.792 312.42) (width 0.25) (layer "F.Cu") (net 27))
 (segment (start 113.792 332.74) (end 113.792 330.2) (width 0.25) (layer "F.Cu") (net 27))
 (segment (start 134.62 356.108) (end 132.842 354.33) (width 0.25) (layer "F.Cu") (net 27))
 (segment (start 113.792 325.12) (end 113.792 322.58) (width 0.25) (layer "F.Cu") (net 27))
 (segment (start 113.792 347.98) (end 116.64 347.98) (width 0.25) (layer "F.Cu") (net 27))
 (segment (start 113.792 317.5) (end 113.792 314.96) (width 0.25) (layer "F.Cu") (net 27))
 (segment (start 138.316002 314.565998) (end 138.316002 319.19) (width 0.25) (layer "F.Cu") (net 27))
 (segment (start 142.748 356.108) (end 134.62 356.108) (width 0.25) (layer "F.Cu") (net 27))
 (segment (start 122.99 354.33) (end 116.65 347.99) (width 0.25) (layer "F.Cu") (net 27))
 (segment (start 113.792 342.9) (end 113.792 340.36) (width 0.25) (layer "F.Cu") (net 27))
 (segment (start 113.792 340.36) (end 113.792 337.82) (width 0.25) (layer "F.Cu") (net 27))
 (segment (start 138.316002 319.19) (end 137.191001 320.315001) (width 0.25) (layer "F.Cu") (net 27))
 (segment (start 113.792 347.98) (end 113.792 345.44) (width 0.25) (layer "F.Cu") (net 27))
 (segment (start 113.792 337.82) (end 113.792 335.28) (width 0.25) (layer "F.Cu") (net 27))
 (segment (start 116.64 347.98) (end 116.65 347.99) (width 0.25) (layer "F.Cu") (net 27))
 (segment (start 113.792 322.58) (end 113.792 320.04) (width 0.25) (layer "F.Cu") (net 27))
 (segment (start 142.748 310.134) (end 138.316002 314.565998) (width 0.25) (layer "F.Cu") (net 27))
 (segment (start 113.792 345.44) (end 113.792 342.9) (width 0.25) (layer "F.Cu") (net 27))
 (segment (start 113.792 335.28) (end 113.792 332.74) (width 0.25) (layer "F.Cu") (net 27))
 (segment (start 113.792 330.2) (end 113.792 327.66) (width 0.25) (layer "F.Cu") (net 27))
 (segment (start 113.792 320.04) (end 113.792 317.5) (width 0.25) (layer "F.Cu") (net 27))
 (segment (start 113.792 313.326998) (end 113.792 320.04) (width 0.25) (layer "B.Cu") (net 27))
 (segment (start 117.751002 319.19) (end 120.581 316.360002) (width 0.25) (layer "B.Cu") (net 27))
 (segment (start 136.066 319.19) (end 117.751002 319.19) (width 0.25) (layer "B.Cu") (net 27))
 (segment (start 123.076002 311.635) (end 122.546001 311.104999) (width 0.25) (layer "B.Cu") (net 27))
 (segment (start 137.191001 320.315001) (end 136.066 319.19) (width 0.25) (layer "B.Cu") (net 27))
 (segment (start 122.491002 316.360002) (end 123.076002 315.775002) (width 0.25) (layer "B.Cu") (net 27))
 (segment (start 122.546001 311.104999) (end 116.013999 311.104999) (width 0.25) (layer "B.Cu") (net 27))
 (segment (start 116.013999 311.104999) (end 113.792 313.326998) (width 0.25) (layer "B.Cu") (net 27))
 (segment (start 120.581 316.360002) (end 122.491002 316.360002) (width 0.25) (layer "B.Cu") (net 27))
 (segment (start 123.076002 315.775002) (end 123.076002 311.635) (width 0.25) (layer "B.Cu") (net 27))
 (segment (start 116.65 335.334) (end 116.65 335.29) (width 0.25) (layer "F.Cu") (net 12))
 (segment (start 121.951001 340.635001) (end 116.65 335.334) (width 0.25) (layer "F.Cu") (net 12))
 (segment (start 121.951001 343.175001) (end 116.65 337.874) (width 0.25) (layer "F.Cu") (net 13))
 (segment (start 116.65 337.874) (end 116.65 337.83) (width 0.25) (layer "F.Cu") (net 13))
 (segment (start 116.65 340.414) (end 116.65 340.37) (width 0.25) (layer "F.Cu") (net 14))
 (segment (start 121.951001 345.715001) (end 116.65 340.414) (width 0.25) (layer "F.Cu") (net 14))
 (segment (start 142.748 315.214) (end 139.71 315.214) (width 0.25) (layer "B.Cu") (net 28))
 (segment (start 139.71 315.214) (end 137.191001 312.695001) (width 0.25) (layer "B.Cu") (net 28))
 (segment (start 121.951001 348.255001) (end 116.65 342.954) (width 0.25) (layer "F.Cu") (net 15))
 (segment (start 116.65 342.954) (end 116.65 342.91) (width 0.25) (layer "F.Cu") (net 15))
 (segment (start 118.040002 346.840002) (end 116.65 345.45) (width 0.25) (layer "B.Cu") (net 16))
 (segment (start 137.191001 348.255001) (end 135.776002 346.840002) (width 0.25) (layer "B.Cu") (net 16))
 (segment (start 135.776002 346.840002) (end 118.040002 346.840002) (width 0.25) (layer "B.Cu") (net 16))
 (segment (start 116.078 356.616) (end 131.064 356.616) (width 0.25) (layer "F.Cu") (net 32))
 (segment (start 131.064 356.616) (end 133.096 358.648) (width 0.25) (layer "F.Cu") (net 32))
 (segment (start 133.096 358.648) (end 142.748 358.648) (width 0.25) (layer "F.Cu") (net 32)))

